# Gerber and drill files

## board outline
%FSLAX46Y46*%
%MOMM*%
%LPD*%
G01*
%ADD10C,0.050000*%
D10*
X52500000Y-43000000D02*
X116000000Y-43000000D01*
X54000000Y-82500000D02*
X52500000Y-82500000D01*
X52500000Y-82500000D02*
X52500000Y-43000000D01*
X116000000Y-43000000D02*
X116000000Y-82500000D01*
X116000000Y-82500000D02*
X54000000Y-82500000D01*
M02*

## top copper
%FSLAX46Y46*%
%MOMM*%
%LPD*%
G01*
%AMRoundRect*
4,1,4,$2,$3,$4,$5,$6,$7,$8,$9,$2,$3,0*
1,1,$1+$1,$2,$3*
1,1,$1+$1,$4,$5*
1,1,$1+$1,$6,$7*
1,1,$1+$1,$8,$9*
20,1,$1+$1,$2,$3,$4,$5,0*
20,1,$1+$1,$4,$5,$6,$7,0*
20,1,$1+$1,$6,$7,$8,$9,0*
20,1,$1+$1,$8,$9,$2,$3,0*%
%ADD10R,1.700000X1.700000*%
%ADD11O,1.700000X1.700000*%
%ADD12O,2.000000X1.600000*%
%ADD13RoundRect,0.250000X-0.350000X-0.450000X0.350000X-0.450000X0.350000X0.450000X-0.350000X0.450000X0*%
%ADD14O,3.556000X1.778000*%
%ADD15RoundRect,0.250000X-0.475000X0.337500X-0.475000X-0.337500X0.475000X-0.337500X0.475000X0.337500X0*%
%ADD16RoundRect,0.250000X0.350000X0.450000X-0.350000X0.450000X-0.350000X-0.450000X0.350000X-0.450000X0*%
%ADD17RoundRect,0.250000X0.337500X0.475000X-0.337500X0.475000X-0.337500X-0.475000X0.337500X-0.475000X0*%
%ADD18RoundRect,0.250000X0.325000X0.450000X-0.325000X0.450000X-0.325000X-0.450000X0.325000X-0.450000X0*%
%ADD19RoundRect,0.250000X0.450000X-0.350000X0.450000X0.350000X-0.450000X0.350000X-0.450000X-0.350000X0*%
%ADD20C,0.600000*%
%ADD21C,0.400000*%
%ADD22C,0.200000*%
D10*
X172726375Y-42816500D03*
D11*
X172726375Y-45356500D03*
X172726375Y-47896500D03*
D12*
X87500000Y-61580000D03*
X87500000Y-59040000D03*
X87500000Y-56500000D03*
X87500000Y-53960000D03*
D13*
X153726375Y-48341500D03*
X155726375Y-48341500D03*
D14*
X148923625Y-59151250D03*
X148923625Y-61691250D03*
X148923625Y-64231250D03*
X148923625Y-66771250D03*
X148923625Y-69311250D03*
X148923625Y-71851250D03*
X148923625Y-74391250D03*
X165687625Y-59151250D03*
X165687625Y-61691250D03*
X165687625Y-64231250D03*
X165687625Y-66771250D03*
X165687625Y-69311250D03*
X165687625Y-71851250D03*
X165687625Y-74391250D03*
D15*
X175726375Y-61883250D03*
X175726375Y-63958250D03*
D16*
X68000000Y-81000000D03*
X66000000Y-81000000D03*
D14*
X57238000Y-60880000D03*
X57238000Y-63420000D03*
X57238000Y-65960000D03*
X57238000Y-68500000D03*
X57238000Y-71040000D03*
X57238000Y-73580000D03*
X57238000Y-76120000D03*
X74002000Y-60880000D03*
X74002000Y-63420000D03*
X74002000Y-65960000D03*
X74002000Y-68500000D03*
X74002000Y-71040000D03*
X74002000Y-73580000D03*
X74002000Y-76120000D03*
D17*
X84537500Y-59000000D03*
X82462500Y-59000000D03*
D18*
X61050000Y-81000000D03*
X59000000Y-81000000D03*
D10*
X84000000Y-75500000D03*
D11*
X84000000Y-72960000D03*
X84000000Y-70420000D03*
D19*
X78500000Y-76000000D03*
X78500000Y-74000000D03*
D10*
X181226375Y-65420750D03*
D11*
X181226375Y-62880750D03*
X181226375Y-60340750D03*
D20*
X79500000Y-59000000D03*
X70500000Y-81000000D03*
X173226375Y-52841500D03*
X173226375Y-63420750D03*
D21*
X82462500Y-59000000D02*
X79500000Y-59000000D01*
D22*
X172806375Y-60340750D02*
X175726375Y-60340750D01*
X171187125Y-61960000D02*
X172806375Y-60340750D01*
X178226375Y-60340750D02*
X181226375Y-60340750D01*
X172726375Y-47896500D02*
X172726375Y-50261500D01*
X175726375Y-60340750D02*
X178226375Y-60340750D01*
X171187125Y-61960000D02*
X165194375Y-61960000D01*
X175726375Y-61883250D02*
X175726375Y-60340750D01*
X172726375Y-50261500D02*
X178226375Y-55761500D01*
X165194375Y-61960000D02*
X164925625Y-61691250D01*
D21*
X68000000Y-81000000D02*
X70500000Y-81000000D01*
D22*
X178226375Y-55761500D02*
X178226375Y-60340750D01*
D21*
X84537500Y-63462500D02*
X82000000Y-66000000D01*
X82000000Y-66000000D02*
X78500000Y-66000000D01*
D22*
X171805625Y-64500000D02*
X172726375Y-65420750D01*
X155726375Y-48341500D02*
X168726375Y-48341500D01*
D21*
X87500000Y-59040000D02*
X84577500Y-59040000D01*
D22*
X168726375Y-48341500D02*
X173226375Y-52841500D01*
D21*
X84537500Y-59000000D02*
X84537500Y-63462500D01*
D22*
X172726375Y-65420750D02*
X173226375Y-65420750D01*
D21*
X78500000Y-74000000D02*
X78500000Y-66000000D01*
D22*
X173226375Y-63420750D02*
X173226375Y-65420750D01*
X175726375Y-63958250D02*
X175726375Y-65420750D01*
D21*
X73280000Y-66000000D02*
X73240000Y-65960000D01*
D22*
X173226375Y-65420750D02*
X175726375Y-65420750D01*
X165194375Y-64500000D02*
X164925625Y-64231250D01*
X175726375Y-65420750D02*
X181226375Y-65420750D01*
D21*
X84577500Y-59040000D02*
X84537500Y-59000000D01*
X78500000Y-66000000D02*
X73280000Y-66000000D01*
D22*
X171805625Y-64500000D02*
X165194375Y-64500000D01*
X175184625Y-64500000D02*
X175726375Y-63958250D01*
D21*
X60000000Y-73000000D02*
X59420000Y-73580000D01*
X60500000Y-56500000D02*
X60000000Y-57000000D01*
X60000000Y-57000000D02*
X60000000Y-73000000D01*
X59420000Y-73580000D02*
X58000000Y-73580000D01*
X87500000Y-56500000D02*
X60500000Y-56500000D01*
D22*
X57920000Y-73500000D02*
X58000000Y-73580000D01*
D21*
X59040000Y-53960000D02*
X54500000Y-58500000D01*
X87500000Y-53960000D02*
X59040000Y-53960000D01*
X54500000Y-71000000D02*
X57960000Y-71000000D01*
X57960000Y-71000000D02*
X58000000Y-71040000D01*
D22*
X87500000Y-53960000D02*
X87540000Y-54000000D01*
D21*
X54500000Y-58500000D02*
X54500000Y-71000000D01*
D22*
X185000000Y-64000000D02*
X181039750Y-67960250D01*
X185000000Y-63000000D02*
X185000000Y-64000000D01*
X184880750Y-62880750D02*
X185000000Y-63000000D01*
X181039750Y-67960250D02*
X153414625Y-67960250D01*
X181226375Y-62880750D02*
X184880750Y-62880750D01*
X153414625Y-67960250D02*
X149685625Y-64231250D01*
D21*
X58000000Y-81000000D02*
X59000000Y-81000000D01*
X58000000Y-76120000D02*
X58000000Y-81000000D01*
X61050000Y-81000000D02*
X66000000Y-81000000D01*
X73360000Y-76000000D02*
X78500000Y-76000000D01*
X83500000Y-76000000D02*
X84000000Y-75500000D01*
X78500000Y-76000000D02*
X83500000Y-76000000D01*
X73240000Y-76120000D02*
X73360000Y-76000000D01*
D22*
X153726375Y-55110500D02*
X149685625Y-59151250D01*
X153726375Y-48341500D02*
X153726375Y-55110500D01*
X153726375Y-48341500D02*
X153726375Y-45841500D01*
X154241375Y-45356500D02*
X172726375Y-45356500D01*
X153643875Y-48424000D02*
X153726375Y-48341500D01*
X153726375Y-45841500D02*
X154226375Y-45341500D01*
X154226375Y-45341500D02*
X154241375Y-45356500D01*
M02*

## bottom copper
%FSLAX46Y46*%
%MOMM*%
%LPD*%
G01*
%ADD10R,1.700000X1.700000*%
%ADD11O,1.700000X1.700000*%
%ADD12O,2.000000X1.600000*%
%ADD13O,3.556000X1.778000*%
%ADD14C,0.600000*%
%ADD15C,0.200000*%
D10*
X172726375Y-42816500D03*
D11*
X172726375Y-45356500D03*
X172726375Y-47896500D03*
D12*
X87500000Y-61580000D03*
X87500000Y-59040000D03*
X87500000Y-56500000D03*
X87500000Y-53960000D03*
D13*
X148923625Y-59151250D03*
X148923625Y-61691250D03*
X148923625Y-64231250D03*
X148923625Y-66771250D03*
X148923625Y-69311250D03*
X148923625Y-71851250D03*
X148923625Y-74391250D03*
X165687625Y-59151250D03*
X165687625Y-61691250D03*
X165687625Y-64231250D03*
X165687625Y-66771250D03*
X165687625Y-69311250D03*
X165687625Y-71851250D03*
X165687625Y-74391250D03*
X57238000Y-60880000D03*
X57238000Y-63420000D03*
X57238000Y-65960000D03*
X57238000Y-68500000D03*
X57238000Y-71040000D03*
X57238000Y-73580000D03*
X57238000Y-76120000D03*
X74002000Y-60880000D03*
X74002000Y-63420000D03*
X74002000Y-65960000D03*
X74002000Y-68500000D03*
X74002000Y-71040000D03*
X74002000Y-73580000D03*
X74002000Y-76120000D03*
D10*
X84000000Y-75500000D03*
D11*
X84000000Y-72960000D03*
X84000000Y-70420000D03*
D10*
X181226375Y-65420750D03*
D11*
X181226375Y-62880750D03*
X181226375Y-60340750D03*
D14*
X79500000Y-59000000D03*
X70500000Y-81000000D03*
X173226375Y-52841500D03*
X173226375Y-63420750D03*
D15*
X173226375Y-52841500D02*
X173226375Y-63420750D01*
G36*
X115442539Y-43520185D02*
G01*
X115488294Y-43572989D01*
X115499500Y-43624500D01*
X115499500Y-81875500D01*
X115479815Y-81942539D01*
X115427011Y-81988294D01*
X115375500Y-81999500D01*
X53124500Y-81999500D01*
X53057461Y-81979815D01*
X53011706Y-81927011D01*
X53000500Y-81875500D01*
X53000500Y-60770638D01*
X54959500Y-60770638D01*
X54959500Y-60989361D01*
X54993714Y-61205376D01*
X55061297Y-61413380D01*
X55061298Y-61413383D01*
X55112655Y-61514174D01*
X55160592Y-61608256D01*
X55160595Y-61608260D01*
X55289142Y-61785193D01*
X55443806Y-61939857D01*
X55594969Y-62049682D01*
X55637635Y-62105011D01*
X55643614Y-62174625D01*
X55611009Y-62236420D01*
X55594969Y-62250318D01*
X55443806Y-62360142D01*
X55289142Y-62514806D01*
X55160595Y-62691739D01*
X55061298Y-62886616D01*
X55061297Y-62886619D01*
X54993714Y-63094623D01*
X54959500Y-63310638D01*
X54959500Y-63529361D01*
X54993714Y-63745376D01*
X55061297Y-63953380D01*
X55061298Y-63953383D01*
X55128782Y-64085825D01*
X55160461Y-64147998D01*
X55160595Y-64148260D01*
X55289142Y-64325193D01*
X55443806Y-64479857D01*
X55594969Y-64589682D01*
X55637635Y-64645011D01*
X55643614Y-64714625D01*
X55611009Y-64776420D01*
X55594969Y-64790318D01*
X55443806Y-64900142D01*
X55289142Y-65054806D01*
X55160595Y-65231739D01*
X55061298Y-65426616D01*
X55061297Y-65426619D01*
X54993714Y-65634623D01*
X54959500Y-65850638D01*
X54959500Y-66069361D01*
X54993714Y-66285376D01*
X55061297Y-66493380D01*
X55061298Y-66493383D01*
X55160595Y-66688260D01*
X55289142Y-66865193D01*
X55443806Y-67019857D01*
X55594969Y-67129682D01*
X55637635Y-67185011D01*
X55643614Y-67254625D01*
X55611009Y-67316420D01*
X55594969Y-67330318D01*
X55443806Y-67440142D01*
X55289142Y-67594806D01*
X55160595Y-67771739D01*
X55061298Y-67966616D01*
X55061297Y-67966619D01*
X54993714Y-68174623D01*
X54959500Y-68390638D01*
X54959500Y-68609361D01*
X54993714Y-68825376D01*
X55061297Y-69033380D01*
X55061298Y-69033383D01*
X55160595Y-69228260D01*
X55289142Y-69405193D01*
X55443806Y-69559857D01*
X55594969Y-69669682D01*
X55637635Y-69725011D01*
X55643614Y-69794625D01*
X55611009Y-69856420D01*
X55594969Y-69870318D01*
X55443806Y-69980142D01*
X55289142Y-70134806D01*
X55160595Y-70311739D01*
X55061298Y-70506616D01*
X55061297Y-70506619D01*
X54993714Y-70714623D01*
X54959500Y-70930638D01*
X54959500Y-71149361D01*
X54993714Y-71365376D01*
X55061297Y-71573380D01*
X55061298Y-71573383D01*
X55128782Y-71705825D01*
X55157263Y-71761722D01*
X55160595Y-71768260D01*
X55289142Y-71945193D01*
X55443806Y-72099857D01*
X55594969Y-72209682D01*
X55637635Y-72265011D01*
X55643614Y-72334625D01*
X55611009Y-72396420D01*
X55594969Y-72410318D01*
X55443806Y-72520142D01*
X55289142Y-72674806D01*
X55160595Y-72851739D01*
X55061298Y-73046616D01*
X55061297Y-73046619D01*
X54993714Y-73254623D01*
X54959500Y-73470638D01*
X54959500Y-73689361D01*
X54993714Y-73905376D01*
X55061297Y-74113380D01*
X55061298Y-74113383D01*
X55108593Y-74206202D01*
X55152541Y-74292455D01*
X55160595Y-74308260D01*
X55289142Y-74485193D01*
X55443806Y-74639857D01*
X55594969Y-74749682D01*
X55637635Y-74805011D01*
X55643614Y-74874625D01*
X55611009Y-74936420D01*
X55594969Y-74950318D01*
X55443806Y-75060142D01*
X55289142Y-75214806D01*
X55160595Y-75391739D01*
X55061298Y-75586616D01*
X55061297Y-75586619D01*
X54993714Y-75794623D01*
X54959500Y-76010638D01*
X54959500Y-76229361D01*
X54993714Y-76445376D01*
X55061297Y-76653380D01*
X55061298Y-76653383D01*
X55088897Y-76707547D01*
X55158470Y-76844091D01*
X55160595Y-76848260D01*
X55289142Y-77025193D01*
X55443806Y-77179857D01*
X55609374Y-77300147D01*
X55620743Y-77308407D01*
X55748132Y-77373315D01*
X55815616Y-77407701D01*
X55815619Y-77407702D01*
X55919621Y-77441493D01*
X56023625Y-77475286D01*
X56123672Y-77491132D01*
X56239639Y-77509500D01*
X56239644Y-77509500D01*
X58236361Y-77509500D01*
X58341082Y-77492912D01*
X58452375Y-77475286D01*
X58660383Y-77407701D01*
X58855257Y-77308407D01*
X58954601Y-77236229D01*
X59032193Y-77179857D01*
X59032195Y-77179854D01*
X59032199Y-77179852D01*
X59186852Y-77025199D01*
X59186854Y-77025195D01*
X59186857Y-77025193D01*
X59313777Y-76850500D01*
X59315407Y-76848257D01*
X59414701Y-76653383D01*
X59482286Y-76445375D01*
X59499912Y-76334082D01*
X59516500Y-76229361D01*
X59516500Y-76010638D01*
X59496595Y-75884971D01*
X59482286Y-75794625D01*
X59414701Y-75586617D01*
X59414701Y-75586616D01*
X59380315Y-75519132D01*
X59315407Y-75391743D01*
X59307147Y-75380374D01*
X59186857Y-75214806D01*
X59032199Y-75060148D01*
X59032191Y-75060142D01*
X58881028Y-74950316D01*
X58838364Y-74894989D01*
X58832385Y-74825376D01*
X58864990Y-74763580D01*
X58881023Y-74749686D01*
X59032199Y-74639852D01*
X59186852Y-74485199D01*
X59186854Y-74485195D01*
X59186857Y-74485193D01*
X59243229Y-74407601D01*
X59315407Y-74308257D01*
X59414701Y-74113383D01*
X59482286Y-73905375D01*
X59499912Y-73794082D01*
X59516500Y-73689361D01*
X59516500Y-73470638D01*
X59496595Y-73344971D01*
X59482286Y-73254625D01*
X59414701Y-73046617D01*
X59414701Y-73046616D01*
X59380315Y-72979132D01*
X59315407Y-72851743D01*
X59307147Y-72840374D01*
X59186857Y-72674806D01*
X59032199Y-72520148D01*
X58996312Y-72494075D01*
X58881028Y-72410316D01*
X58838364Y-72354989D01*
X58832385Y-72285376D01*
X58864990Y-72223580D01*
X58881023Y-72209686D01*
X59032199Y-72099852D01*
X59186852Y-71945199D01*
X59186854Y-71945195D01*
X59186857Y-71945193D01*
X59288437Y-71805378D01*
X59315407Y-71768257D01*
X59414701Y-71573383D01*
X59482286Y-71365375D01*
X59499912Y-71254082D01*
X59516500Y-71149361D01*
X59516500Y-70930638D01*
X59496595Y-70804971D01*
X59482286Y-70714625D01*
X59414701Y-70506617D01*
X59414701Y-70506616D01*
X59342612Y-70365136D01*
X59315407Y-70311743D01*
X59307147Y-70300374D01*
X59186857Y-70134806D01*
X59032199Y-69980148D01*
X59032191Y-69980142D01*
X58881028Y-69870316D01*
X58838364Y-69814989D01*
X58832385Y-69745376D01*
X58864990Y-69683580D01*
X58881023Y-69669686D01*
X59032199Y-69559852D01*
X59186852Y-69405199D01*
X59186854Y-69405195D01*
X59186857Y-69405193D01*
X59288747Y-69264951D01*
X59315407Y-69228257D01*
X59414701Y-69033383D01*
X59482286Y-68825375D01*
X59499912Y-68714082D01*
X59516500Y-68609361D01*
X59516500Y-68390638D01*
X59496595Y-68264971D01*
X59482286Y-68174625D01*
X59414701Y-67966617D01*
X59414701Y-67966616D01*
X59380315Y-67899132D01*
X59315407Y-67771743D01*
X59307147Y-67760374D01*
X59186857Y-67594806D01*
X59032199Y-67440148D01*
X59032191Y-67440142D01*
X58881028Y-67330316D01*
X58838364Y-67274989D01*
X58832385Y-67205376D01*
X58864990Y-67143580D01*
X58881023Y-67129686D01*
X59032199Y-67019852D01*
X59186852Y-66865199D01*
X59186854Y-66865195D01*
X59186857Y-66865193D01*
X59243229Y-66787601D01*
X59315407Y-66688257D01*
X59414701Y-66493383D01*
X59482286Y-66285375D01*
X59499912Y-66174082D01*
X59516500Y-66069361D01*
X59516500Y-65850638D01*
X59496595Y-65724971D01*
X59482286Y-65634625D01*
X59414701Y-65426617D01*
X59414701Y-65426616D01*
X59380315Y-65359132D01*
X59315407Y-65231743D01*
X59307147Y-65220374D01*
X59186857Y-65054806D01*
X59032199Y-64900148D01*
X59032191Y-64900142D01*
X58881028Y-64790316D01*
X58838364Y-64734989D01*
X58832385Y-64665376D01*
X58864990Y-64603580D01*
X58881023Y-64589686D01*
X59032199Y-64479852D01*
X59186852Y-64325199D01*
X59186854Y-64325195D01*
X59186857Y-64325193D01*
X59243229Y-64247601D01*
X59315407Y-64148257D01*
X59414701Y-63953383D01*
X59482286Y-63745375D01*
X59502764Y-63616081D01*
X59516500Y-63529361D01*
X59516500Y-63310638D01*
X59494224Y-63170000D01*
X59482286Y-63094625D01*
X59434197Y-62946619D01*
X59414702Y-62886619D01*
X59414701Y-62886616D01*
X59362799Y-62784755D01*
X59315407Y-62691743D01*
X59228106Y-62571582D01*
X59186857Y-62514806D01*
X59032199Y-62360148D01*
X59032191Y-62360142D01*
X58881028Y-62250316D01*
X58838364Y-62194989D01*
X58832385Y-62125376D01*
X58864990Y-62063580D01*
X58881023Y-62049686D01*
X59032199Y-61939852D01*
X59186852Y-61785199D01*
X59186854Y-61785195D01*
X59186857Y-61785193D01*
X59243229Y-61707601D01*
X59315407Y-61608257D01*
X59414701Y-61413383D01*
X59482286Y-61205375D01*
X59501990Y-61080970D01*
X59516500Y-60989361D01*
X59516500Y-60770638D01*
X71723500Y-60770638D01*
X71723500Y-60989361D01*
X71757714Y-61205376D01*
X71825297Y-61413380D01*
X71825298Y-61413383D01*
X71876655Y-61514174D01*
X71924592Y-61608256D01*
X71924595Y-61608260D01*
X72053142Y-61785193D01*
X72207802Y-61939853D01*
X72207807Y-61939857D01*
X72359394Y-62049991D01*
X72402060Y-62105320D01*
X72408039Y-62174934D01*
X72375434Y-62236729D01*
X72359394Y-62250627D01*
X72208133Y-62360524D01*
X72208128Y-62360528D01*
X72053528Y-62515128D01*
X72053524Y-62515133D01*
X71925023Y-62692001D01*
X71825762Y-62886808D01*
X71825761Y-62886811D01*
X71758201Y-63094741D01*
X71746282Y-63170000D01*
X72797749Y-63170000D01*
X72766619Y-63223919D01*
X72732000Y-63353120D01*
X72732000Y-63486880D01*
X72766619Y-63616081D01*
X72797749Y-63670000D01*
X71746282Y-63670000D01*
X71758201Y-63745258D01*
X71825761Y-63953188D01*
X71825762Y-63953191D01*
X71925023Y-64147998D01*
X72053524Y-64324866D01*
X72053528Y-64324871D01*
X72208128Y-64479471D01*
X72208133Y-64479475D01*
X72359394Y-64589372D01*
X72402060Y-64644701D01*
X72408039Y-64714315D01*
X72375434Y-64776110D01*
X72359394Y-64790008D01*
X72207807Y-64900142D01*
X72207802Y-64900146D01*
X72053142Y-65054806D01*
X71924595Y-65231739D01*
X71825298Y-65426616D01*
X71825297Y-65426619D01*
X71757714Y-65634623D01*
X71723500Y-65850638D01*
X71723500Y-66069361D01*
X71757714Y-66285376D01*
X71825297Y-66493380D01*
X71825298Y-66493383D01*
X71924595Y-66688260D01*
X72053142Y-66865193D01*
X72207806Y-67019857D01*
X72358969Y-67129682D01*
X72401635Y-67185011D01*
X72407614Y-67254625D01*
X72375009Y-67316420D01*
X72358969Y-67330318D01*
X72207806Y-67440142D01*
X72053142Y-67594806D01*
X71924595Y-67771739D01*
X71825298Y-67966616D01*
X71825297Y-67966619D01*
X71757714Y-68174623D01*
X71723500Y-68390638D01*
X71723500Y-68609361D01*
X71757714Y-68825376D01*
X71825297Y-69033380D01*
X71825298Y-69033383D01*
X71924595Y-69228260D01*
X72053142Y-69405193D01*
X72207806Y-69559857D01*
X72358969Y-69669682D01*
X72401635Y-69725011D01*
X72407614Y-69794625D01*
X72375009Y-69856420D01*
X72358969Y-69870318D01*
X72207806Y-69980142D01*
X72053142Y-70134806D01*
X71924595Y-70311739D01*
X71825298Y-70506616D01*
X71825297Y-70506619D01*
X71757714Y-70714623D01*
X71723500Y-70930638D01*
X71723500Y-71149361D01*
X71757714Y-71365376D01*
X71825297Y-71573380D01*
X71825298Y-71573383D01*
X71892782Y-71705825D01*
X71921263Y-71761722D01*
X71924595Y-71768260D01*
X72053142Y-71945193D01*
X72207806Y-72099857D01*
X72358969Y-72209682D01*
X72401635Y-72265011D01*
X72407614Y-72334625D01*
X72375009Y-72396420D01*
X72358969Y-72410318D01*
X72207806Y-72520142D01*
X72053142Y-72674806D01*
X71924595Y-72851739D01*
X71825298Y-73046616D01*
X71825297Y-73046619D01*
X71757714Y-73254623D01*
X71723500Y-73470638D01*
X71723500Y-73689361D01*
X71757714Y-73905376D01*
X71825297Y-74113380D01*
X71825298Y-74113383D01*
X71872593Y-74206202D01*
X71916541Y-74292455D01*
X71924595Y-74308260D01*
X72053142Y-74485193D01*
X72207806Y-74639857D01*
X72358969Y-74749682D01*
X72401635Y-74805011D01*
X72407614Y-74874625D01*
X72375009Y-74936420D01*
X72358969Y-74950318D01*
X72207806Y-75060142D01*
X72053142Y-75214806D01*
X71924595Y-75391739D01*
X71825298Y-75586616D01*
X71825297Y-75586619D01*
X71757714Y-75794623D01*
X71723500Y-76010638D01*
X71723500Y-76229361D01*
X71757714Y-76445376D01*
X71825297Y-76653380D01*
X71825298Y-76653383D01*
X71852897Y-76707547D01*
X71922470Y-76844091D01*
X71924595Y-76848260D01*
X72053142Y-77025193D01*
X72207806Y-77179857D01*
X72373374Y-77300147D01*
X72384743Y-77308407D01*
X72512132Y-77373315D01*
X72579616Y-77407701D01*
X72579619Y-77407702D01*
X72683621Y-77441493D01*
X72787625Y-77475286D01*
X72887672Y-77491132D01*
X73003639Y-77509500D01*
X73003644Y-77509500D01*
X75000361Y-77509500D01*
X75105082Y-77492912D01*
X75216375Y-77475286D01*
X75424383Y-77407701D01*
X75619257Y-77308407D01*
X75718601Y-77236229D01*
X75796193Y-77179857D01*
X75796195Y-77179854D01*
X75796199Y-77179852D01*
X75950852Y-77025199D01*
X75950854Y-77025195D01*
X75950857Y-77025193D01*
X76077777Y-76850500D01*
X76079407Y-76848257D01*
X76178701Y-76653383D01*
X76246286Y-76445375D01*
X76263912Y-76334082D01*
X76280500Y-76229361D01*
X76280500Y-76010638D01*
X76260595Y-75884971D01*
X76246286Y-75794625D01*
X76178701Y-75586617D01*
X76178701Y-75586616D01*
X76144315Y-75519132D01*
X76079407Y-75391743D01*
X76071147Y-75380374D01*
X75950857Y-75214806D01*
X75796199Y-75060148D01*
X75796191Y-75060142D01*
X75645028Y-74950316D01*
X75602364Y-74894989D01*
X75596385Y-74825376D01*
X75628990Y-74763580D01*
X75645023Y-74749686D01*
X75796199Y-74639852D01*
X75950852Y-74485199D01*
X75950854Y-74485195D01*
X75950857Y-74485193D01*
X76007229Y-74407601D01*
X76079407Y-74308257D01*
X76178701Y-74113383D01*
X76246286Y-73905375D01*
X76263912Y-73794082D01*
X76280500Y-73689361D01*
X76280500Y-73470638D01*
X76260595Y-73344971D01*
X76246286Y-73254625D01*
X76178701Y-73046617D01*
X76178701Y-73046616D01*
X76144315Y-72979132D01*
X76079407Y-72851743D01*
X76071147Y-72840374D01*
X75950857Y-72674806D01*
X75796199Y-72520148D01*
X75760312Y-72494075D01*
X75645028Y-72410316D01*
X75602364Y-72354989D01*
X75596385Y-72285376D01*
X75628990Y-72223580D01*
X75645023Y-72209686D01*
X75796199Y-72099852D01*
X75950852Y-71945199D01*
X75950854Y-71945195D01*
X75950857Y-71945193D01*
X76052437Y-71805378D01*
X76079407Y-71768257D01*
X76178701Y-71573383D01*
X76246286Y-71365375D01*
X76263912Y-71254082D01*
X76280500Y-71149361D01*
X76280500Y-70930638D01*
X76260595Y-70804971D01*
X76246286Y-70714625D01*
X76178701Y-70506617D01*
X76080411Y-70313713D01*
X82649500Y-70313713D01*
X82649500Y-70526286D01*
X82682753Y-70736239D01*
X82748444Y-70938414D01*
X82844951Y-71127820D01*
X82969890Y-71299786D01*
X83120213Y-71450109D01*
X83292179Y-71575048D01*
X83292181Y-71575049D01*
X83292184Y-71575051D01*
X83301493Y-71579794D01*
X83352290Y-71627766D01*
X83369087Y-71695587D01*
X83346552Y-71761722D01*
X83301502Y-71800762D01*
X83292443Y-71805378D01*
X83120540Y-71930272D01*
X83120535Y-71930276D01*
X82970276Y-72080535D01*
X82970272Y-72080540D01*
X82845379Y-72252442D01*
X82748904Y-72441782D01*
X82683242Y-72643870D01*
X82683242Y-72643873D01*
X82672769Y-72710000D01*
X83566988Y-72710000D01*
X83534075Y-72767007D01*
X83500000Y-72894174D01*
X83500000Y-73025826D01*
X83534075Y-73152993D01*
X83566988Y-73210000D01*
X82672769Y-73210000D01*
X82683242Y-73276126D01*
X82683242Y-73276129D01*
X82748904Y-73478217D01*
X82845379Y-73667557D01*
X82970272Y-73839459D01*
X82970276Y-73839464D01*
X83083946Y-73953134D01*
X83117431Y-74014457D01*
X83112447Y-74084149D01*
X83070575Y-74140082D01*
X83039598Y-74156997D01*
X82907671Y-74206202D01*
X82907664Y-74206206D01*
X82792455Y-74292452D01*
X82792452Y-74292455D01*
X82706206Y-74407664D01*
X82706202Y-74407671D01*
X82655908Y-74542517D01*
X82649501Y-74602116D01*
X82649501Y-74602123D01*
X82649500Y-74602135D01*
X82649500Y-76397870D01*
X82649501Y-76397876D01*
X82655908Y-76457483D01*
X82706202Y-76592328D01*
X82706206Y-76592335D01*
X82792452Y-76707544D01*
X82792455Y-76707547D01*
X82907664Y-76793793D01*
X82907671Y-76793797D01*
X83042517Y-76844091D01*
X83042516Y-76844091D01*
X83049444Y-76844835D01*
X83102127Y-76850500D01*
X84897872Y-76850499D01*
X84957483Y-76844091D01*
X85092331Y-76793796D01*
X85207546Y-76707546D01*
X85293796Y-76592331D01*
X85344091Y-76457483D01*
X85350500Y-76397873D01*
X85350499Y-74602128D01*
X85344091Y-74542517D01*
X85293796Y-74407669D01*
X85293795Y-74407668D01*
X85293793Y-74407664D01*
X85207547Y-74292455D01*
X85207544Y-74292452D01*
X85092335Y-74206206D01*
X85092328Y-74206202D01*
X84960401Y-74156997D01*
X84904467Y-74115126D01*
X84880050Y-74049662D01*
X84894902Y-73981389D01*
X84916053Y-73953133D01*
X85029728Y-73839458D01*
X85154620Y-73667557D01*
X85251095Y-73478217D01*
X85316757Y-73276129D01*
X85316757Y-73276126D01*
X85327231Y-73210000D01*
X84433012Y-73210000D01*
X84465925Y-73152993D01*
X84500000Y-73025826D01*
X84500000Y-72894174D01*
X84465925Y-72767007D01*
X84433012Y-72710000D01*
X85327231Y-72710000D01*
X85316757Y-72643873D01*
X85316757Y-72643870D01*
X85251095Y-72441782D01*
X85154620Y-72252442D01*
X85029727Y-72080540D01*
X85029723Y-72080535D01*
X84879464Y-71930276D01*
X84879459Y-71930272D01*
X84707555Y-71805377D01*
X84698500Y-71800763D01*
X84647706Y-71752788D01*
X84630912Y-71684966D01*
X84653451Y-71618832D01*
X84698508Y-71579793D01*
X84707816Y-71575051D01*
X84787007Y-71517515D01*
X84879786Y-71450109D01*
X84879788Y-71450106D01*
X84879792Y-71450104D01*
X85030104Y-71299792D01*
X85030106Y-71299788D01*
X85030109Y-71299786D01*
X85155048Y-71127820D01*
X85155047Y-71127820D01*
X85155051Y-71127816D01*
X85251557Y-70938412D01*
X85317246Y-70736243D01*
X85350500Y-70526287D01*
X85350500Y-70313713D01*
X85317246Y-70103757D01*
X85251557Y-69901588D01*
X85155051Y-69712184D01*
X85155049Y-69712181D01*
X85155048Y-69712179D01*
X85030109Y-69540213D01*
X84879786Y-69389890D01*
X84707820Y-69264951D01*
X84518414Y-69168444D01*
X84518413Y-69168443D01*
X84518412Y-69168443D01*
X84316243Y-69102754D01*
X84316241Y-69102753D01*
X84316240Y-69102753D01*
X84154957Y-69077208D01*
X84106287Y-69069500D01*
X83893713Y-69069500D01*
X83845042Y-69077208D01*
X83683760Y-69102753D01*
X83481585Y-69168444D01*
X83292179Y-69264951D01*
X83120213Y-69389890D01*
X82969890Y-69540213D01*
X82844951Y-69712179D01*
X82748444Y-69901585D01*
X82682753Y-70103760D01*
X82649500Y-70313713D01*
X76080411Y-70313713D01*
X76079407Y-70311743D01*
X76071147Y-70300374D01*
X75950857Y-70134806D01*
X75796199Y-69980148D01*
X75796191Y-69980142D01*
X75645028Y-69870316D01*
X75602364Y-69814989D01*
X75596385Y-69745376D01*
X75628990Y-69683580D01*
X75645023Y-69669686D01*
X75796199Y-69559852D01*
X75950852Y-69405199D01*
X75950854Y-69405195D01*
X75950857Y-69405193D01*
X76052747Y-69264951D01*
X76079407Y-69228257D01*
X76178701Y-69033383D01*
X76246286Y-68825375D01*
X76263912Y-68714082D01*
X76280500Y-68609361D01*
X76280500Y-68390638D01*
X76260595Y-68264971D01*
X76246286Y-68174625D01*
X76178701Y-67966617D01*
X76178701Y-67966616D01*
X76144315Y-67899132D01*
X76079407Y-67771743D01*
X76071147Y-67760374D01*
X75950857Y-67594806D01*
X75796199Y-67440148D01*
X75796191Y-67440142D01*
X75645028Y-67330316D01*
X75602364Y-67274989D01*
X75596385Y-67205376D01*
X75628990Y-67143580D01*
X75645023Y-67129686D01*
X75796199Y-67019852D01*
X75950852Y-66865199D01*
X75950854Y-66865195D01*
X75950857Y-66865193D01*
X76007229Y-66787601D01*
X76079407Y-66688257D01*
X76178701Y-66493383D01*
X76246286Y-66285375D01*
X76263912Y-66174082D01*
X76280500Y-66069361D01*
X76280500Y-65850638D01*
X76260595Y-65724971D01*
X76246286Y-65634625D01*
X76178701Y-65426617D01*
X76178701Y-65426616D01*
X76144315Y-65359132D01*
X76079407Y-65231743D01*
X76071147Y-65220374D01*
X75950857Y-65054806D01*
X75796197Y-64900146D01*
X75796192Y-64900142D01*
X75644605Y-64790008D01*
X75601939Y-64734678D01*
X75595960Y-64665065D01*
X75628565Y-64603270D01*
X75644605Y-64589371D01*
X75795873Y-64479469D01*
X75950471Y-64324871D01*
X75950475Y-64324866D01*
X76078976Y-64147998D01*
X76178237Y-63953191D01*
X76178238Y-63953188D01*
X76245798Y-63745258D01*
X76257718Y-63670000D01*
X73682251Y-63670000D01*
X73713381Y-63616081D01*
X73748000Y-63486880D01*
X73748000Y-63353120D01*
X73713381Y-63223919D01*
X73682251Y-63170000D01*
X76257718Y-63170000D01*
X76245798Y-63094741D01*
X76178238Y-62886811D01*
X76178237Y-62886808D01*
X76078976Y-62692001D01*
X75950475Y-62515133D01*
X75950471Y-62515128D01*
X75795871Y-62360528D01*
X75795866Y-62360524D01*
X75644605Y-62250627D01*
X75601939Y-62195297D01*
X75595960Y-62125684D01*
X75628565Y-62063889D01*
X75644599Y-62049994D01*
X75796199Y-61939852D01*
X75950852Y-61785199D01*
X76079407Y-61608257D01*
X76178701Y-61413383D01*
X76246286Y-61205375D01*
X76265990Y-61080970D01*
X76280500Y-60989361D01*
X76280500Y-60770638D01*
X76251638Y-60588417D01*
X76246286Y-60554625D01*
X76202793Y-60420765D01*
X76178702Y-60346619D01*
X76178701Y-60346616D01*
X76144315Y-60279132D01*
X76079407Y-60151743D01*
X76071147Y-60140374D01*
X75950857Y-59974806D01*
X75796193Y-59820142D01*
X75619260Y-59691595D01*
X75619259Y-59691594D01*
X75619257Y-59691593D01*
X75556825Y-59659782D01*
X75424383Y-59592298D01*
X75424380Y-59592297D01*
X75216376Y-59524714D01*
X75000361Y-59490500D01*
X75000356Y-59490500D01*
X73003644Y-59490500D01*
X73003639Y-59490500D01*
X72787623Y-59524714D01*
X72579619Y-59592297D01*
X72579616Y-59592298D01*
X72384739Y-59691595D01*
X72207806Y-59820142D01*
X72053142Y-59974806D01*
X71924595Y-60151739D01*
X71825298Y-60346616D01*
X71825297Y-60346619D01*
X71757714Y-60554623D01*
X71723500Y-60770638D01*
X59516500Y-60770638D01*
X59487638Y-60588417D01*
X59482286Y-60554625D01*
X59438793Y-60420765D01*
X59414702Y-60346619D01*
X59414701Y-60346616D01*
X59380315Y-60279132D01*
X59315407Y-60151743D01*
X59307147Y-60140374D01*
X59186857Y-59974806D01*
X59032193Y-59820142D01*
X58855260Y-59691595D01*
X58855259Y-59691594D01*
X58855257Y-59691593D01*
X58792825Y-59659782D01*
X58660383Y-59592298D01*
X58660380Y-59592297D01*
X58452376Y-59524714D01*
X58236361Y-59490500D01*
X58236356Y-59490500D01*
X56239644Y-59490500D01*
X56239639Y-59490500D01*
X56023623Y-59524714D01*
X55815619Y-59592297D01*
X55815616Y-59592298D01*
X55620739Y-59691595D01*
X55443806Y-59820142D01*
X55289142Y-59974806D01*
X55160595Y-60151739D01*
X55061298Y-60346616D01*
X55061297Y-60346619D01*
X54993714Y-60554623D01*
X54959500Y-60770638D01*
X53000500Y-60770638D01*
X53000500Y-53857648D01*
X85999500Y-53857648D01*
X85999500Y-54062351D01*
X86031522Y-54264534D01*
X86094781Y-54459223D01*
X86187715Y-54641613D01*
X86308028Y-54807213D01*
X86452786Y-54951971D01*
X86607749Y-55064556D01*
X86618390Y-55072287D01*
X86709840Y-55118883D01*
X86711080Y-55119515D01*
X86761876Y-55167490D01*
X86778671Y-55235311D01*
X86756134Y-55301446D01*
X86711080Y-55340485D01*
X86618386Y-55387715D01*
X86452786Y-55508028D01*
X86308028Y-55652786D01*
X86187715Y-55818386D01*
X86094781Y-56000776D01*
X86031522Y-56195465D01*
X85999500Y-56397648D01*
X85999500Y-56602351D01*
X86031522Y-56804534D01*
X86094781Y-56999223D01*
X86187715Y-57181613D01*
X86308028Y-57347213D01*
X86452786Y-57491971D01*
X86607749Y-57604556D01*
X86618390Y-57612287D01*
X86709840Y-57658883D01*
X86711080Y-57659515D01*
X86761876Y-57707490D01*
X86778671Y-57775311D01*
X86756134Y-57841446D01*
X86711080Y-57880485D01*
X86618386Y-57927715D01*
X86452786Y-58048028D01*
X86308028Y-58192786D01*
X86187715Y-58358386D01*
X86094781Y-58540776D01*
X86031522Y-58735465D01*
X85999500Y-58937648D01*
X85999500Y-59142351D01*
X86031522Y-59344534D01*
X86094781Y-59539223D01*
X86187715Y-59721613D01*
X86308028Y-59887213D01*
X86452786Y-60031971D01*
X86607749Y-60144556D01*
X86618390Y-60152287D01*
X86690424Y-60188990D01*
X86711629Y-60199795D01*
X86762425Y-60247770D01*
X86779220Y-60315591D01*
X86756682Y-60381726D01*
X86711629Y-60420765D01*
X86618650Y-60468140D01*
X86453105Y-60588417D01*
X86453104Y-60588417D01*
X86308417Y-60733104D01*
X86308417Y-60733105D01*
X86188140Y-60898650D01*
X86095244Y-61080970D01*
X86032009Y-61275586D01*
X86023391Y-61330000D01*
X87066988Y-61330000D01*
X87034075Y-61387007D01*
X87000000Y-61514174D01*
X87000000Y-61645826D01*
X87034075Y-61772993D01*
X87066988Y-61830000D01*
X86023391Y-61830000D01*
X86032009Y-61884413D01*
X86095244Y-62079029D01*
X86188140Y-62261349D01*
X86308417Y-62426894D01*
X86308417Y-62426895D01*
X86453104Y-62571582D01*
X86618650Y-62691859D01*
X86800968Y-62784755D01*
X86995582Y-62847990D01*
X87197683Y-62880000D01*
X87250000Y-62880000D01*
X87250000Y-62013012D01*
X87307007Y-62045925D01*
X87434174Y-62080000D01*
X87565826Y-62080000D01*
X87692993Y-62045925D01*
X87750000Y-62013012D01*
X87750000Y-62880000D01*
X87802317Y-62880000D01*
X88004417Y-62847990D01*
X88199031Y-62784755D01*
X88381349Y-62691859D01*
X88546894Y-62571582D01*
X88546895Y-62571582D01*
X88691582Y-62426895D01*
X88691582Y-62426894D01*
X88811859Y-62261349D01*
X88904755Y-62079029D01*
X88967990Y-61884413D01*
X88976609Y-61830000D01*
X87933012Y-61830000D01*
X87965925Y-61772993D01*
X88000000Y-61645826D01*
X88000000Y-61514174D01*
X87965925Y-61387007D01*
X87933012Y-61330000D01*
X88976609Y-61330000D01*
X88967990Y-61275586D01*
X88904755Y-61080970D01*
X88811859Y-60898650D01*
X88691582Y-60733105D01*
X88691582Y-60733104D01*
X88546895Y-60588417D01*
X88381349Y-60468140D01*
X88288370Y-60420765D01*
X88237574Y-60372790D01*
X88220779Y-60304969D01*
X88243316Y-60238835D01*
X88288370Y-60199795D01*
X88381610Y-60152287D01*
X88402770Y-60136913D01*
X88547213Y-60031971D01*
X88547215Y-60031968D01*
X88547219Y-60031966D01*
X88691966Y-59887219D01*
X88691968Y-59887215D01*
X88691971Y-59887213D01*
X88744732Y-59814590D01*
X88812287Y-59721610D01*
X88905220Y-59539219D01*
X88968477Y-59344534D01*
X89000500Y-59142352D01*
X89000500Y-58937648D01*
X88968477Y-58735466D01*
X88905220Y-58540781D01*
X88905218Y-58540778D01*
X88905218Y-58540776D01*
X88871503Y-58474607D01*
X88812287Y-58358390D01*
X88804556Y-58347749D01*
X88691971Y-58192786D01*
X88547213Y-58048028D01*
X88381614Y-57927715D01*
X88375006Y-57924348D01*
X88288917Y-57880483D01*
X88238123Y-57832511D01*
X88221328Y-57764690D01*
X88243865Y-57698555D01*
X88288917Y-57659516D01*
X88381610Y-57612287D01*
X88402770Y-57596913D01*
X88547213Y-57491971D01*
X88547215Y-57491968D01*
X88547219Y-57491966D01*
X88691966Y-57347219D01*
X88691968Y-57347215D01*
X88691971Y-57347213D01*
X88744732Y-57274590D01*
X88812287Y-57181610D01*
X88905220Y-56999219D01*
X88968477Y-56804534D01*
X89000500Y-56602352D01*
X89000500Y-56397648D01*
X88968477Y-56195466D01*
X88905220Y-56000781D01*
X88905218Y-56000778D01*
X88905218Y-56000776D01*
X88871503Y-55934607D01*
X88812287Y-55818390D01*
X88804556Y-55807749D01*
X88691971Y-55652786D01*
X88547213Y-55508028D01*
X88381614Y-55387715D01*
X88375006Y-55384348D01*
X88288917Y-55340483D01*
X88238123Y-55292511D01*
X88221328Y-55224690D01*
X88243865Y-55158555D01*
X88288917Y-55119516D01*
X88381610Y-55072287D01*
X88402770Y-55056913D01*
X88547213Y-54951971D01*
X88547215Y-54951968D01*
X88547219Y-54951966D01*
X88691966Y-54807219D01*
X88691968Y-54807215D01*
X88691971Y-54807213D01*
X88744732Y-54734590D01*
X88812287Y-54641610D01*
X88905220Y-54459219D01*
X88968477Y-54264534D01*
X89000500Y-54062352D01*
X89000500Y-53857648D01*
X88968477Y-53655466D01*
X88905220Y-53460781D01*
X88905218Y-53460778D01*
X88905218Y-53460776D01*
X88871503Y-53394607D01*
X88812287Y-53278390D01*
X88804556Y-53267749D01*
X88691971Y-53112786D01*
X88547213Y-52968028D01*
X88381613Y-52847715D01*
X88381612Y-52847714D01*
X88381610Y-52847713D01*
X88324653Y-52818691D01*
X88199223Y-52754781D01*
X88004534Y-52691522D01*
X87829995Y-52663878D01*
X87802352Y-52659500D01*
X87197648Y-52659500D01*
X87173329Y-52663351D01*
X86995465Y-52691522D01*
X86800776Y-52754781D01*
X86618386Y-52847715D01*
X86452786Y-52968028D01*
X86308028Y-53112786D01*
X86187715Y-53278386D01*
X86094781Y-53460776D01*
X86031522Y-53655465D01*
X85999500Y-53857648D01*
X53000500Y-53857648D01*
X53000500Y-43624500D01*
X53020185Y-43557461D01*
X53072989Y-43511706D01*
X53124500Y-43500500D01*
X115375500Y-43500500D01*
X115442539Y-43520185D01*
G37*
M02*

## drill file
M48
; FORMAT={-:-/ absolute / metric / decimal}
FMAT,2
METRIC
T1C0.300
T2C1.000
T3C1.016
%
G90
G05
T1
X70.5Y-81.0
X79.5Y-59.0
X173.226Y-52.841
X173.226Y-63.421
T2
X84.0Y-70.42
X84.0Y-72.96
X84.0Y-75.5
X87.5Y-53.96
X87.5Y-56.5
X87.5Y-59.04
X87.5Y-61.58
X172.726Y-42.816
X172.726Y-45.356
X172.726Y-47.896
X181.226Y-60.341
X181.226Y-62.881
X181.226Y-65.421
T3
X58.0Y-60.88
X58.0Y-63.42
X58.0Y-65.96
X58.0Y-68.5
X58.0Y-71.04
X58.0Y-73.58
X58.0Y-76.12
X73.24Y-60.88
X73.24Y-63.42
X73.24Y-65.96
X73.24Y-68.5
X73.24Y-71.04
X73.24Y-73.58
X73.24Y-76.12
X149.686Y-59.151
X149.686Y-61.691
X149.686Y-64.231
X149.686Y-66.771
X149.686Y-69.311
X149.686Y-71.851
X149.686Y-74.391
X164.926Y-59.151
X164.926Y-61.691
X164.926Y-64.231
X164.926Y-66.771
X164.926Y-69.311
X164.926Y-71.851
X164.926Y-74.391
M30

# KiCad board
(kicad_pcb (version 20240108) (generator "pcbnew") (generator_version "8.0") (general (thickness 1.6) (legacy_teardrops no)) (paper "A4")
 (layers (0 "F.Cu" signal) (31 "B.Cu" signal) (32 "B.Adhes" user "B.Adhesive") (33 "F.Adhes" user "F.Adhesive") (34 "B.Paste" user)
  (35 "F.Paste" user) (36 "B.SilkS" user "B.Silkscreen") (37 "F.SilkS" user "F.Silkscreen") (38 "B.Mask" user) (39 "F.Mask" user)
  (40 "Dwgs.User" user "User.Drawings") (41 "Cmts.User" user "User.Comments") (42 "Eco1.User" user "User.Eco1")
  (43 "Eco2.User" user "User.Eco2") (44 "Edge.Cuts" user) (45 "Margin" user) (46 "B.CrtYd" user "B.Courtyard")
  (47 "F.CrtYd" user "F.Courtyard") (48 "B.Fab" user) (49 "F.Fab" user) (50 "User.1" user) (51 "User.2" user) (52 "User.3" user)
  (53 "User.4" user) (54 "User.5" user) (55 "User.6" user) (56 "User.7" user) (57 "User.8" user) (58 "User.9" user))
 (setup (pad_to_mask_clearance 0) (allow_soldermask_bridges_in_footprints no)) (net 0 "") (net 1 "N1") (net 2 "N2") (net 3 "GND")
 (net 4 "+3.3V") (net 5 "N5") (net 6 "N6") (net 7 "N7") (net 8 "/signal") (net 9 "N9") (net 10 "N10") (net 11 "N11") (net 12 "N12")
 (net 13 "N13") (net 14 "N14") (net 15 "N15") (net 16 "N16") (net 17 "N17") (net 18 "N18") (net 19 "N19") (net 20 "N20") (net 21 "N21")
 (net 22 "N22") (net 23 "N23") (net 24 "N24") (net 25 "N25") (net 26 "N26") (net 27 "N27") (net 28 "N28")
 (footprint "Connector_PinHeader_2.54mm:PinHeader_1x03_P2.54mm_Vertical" (layer "F.Cu") (at 172.726375 42.8165)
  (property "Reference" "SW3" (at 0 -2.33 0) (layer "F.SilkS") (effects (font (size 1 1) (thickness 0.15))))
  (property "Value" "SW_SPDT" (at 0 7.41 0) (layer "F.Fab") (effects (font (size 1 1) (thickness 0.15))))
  (pad "1" thru_hole rect (at 0 0) (size 1.7 1.7) (drill 1) (layers "*.Cu" "*.Mask") (remove_unused_layers no) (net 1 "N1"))
  (pad "2" thru_hole oval (at 0 2.54) (size 1.7 1.7) (drill 1) (layers "*.Cu" "*.Mask") (remove_unused_layers no) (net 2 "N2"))
  (pad "3" thru_hole oval (at 0 5.08) (size 1.7 1.7) (drill 1) (layers "*.Cu" "*.Mask") (remove_unused_layers no) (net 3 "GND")))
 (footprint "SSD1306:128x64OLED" (layer "F.Cu") (at 98.1 57.96 90)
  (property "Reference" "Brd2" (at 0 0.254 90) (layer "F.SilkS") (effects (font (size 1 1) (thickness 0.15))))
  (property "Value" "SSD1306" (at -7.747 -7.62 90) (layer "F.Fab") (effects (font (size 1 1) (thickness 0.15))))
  (pad "1" thru_hole oval (at -3.62 -10.6 180) (size 2 1.6) (drill 1) (layers "*.Cu" "*.Mask") (remove_unused_layers no) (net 3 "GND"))
  (pad "2" thru_hole oval (at -1.08 -10.6 180) (size 2 1.6) (drill 1) (layers "*.Cu" "*.Mask") (remove_unused_layers no) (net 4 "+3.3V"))
  (pad "3" thru_hole oval (at 1.46 -10.6 180) (size 2 1.6) (drill 1) (layers "*.Cu" "*.Mask") (remove_unused_layers no) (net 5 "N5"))
  (pad "4" thru_hole oval (at 4 -10.6 180) (size 2 1.6) (drill 1) (layers "*.Cu" "*.Mask") (remove_unused_layers no) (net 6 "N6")))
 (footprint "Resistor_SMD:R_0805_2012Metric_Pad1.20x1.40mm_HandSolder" (layer "F.Cu") (at 154.726375 48.3415)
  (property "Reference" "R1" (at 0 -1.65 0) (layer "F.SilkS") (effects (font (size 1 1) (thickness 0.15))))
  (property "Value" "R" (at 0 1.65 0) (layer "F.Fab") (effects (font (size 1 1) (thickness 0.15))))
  (pad "1" smd roundrect (at -1 0) (size 1.2 1.4) (layers "F.Cu" "F.Paste" "F.Mask") (roundrect_rratio 0.208333) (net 2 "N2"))
  (pad "2" smd roundrect (at 1 0) (size 1.2 1.4) (layers "F.Cu" "F.Paste" "F.Mask") (roundrect_rratio 0.208333) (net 4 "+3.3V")))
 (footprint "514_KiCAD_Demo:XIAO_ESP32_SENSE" (layer "F.Cu") (at 157.305625 66.77125)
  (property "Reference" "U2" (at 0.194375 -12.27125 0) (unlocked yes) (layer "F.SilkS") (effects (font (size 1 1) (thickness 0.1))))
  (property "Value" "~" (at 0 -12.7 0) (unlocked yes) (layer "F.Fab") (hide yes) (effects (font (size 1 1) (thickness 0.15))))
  (pad "1" thru_hole oval (at -7.62 -7.62) (size 3.556 1.778) (drill 1.016 (offset -0.762 0)) (layers "*.Cu" "*.Mask")
   (remove_unused_layers no) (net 2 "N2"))
  (pad "2" thru_hole oval (at -7.62 -5.08) (size 3.556 1.778) (drill 1.016 (offset -0.762 0)) (layers "*.Cu" "*.Mask")
   (remove_unused_layers no) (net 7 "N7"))
  (pad "3" thru_hole oval (at -7.62 -2.54) (size 3.556 1.778) (drill 1.016 (offset -0.762 0)) (layers "*.Cu" "*.Mask")
   (remove_unused_layers no) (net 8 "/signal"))
  (pad "4" thru_hole oval (at -7.62 0) (size 3.556 1.778) (drill 1.016 (offset -0.762 0)) (layers "*.Cu" "*.Mask") (remove_unused_layers no)
   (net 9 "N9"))
  (pad "5" thru_hole oval (at -7.62 2.54) (size 3.556 1.778) (drill 1.016 (offset -0.762 0)) (layers "*.Cu" "*.Mask")
   (remove_unused_layers no) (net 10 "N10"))
  (pad "6" thru_hole oval (at -7.62 5.08) (size 3.556 1.778) (drill 1.016 (offset -0.762 0)) (layers "*.Cu" "*.Mask")
   (remove_unused_layers no) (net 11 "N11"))
  (pad "7" thru_hole oval (at -7.62 7.62) (size 3.556 1.778) (drill 1.016 (offset -0.762 0)) (layers "*.Cu" "*.Mask")
   (remove_unused_layers no) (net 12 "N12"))
  (pad "8" thru_hole oval (at 7.62 -7.62) (size 3.556 1.778) (drill 1.016 (offset 0.762 0)) (layers "*.Cu" "*.Mask")
   (remove_unused_layers no) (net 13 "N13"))
  (pad "9" thru_hole oval (at 7.62 -5.08) (size 3.556 1.778) (drill 1.016 (offset 0.762 0)) (layers "*.Cu" "*.Mask")
   (remove_unused_layers no) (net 3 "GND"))
  (pad "10" thru_hole oval (at 7.62 -2.54) (size 3.556 1.778) (drill 1.016 (offset 0.762 0)) (layers "*.Cu" "*.Mask")
   (remove_unused_layers no) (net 4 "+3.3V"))
  (pad "11" thru_hole oval (at 7.62 0) (size 3.556 1.778) (drill 1.016 (offset 0.762 0)) (layers "*.Cu" "*.Mask") (remove_unused_layers no)
   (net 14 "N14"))
  (pad "12" thru_hole oval (at 7.62 2.54) (size 3.556 1.778) (drill 1.016 (offset 0.762 0)) (layers "*.Cu" "*.Mask")
   (remove_unused_layers no) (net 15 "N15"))
  (pad "13" thru_hole oval (at 7.62 5.08) (size 3.556 1.778) (drill 1.016 (offset 0.762 0)) (layers "*.Cu" "*.Mask")
   (remove_unused_layers no) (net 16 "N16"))
  (pad "14" thru_hole oval (at 7.62 7.62) (size 3.556 1.778) (drill 1.016 (offset 0.762 0)) (layers "*.Cu" "*.Mask")
   (remove_unused_layers no) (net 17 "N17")))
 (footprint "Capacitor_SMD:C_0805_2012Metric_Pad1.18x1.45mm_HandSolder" (layer "F.Cu") (at 175.726375 62.92075 -90)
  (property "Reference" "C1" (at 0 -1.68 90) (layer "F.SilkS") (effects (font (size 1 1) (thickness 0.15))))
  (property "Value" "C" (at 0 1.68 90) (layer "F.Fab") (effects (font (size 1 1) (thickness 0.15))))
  (pad "1" smd roundrect (at -1.0375 0 270) (size 1.175 1.45) (layers "F.Cu" "F.Paste" "F.Mask") (roundrect_rratio 0.212766) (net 3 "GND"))
  (pad "2" smd roundrect (at 1.0375 0 270) (size 1.175 1.45) (layers "F.Cu" "F.Paste" "F.Mask") (roundrect_rratio 0.212766) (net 4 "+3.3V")))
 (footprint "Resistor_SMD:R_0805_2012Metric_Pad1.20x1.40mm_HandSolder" (layer "F.Cu") (at 67 81 180)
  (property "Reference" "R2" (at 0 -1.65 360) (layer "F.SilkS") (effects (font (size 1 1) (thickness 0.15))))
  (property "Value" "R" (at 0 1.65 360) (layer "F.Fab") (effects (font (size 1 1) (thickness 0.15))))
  (pad "1" smd roundrect (at -1 0 180) (size 1.2 1.4) (layers "F.Cu" "F.Paste" "F.Mask") (roundrect_rratio 0.208333) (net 3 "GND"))
  (pad "2" smd roundrect (at 1 0 180) (size 1.2 1.4) (layers "F.Cu" "F.Paste" "F.Mask") (roundrect_rratio 0.208333) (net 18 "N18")))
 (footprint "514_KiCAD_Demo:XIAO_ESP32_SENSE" (layer "F.Cu") (at 65.62 68.5)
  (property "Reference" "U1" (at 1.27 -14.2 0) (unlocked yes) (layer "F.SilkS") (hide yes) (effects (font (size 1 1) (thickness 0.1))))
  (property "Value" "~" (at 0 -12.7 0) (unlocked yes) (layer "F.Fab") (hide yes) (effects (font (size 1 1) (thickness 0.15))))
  (pad "1" thru_hole oval (at -7.62 -7.62) (size 3.556 1.778) (drill 1.016 (offset -0.762 0)) (layers "*.Cu" "*.Mask")
   (remove_unused_layers no) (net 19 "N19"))
  (pad "2" thru_hole oval (at -7.62 -5.08) (size 3.556 1.778) (drill 1.016 (offset -0.762 0)) (layers "*.Cu" "*.Mask")
   (remove_unused_layers no) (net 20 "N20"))
  (pad "3" thru_hole oval (at -7.62 -2.54) (size 3.556 1.778) (drill 1.016 (offset -0.762 0)) (layers "*.Cu" "*.Mask")
   (remove_unused_layers no) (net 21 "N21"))
  (pad "4" thru_hole oval (at -7.62 0) (size 3.556 1.778) (drill 1.016 (offset -0.762 0)) (layers "*.Cu" "*.Mask") (remove_unused_layers no)
   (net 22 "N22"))
  (pad "5" thru_hole oval (at -7.62 2.54) (size 3.556 1.778) (drill 1.016 (offset -0.762 0)) (layers "*.Cu" "*.Mask")
   (remove_unused_layers no) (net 6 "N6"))
  (pad "6" thru_hole oval (at -7.62 5.08) (size 3.556 1.778) (drill 1.016 (offset -0.762 0)) (layers "*.Cu" "*.Mask")
   (remove_unused_layers no) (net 5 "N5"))
  (pad "7" thru_hole oval (at -7.62 7.62) (size 3.556 1.778) (drill 1.016 (offset -0.762 0)) (layers "*.Cu" "*.Mask")
   (remove_unused_layers no) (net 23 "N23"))
  (pad "8" thru_hole oval (at 7.62 -7.62) (size 3.556 1.778) (drill 1.016 (offset 0.762 0)) (layers "*.Cu" "*.Mask")
   (remove_unused_layers no) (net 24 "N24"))
  (pad "9" thru_hole oval (at 7.62 -5.08) (size 3.556 1.778) (drill 1.016 (offset 0.762 0)) (layers "*.Cu" "*.Mask")
   (remove_unused_layers no) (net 3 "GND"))
  (pad "10" thru_hole oval (at 7.62 -2.54) (size 3.556 1.778) (drill 1.016 (offset 0.762 0)) (layers "*.Cu" "*.Mask")
   (remove_unused_layers no) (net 4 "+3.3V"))
  (pad "11" thru_hole oval (at 7.62 0) (size 3.556 1.778) (drill 1.016 (offset 0.762 0)) (layers "*.Cu" "*.Mask") (remove_unused_layers no)
   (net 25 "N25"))
  (pad "12" thru_hole oval (at 7.62 2.54) (size 3.556 1.778) (drill 1.016 (offset 0.762 0)) (layers "*.Cu" "*.Mask")
   (remove_unused_layers no) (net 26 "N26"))
  (pad "13" thru_hole oval (at 7.62 5.08) (size 3.556 1.778) (drill 1.016 (offset 0.762 0)) (layers "*.Cu" "*.Mask")
   (remove_unused_layers no) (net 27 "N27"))
  (pad "14" thru_hole oval (at 7.62 7.62) (size 3.556 1.778) (drill 1.016 (offset 0.762 0)) (layers "*.Cu" "*.Mask")
   (remove_unused_layers no) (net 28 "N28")))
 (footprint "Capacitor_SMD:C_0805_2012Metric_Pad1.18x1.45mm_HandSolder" (layer "F.Cu") (at 83.5 59 180)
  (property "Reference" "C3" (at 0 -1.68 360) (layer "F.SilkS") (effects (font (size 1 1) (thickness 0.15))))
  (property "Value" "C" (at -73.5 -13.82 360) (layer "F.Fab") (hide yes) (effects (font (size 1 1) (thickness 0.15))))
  (pad "1" smd roundrect (at -1.0375 0 180) (size 1.175 1.45) (layers "F.Cu" "F.Paste" "F.Mask") (roundrect_rratio 0.212766) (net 4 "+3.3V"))
  (pad "2" smd roundrect (at 1.0375 0 180) (size 1.175 1.45) (layers "F.Cu" "F.Paste" "F.Mask") (roundrect_rratio 0.212766) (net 3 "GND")))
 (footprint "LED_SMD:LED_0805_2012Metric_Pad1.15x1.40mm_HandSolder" (layer "F.Cu") (at 60.025 81 180)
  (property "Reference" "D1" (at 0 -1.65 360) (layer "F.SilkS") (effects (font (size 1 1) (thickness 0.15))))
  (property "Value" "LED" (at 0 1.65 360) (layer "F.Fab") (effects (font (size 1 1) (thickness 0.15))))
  (pad "1" smd roundrect (at -1.025 0 180) (size 1.15 1.4) (layers "F.Cu" "F.Paste" "F.Mask") (roundrect_rratio 0.217391) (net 18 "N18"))
  (pad "2" smd roundrect (at 1.025 0 180) (size 1.15 1.4) (layers "F.Cu" "F.Paste" "F.Mask") (roundrect_rratio 0.217391) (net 23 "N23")))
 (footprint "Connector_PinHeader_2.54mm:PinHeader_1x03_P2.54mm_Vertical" (layer "F.Cu") (at 84 75.5 180)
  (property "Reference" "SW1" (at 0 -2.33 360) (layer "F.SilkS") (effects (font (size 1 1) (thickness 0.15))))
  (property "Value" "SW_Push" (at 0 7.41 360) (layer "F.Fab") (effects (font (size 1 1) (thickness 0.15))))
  (pad "1" thru_hole rect (at 0 0 180) (size 1.7 1.7) (drill 1) (layers "*.Cu" "*.Mask") (remove_unused_layers no) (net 28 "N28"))
  (pad "2" thru_hole oval (at 0 2.54 180) (size 1.7 1.7) (drill 1) (layers "*.Cu" "*.Mask") (remove_unused_layers no) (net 3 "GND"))
  (pad "3" thru_hole oval (at 0 5.08 180) (size 1.7 1.7) (drill 1) (layers "*.Cu" "*.Mask") (remove_unused_layers no)))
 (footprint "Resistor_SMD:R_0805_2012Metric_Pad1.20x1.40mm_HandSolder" (layer "F.Cu") (at 78.5 75 90)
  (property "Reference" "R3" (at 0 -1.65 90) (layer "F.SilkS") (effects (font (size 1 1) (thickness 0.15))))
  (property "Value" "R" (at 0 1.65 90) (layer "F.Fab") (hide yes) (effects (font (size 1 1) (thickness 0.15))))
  (pad "1" smd roundrect (at -1 0 90) (size 1.2 1.4) (layers "F.Cu" "F.Paste" "F.Mask") (roundrect_rratio 0.208333) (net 28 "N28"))
  (pad "2" smd roundrect (at 1 0 90) (size 1.2 1.4) (layers "F.Cu" "F.Paste" "F.Mask") (roundrect_rratio 0.208333) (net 4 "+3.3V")))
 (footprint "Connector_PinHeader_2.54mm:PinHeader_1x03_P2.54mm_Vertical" (layer "F.Cu") (at 181.226375 65.42075 180)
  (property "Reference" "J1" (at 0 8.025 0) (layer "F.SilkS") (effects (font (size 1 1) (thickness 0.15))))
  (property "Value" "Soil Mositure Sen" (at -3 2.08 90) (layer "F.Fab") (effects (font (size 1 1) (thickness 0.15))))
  (pad "1" thru_hole rect (at 0 0 180) (size 1.7 1.7) (drill 1) (layers "*.Cu" "*.Mask") (remove_unused_layers no) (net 4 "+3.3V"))
  (pad "2" thru_hole oval (at 0 2.54 180) (size 1.7 1.7) (drill 1) (layers "*.Cu" "*.Mask") (remove_unused_layers no) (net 8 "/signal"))
  (pad "3" thru_hole oval (at 0 5.08 180) (size 1.7 1.7) (drill 1) (layers "*.Cu" "*.Mask") (remove_unused_layers no) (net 3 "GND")))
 (gr_line (start 52.5 43) (end 116 43) (stroke (width 0.05) (type default)) (layer "Edge.Cuts"))
 (gr_line (start 54 82.5) (end 52.5 82.5) (stroke (width 0.05) (type default)) (layer "Edge.Cuts"))
 (gr_line (start 52.5 82.5) (end 52.5 43) (stroke (width 0.05) (type default)) (layer "Edge.Cuts"))
 (gr_line (start 116 43) (end 116 82.5) (stroke (width 0.05) (type default)) (layer "Edge.Cuts"))
 (gr_line (start 116 82.5) (end 54 82.5) (stroke (width 0.05) (type default)) (layer "Edge.Cuts"))
 (segment (start 82.4625 59) (end 79.5 59) (width 0.4) (layer "F.Cu") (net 3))
 (segment (start 172.806375 60.34075) (end 175.726375 60.34075) (width 0.2) (layer "F.Cu") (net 3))
 (segment (start 171.187125 61.96) (end 172.806375 60.34075) (width 0.2) (layer "F.Cu") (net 3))
 (segment (start 178.226375 60.34075) (end 181.226375 60.34075) (width 0.2) (layer "F.Cu") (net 3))
 (segment (start 172.726375 47.8965) (end 172.726375 50.2615) (width 0.2) (layer "F.Cu") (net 3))
 (segment (start 175.726375 60.34075) (end 178.226375 60.34075) (width 0.2) (layer "F.Cu") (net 3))
 (segment (start 171.187125 61.96) (end 165.194375 61.96) (width 0.2) (layer "F.Cu") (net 3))
 (segment (start 175.726375 61.88325) (end 175.726375 60.34075) (width 0.2) (layer "F.Cu") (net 3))
 (segment (start 172.726375 50.2615) (end 178.226375 55.7615) (width 0.2) (layer "F.Cu") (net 3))
 (segment (start 165.194375 61.96) (end 164.925625 61.69125) (width 0.2) (layer "F.Cu") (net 3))
 (segment (start 68 81) (end 70.5 81) (width 0.4) (layer "F.Cu") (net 3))
 (segment (start 178.226375 55.7615) (end 178.226375 60.34075) (width 0.2) (layer "F.Cu") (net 3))
 (via (at 79.5 59) (size 0.6) (drill 0.3) (layers "F.Cu" "B.Cu") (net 3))
 (via (at 70.5 81) (size 0.6) (drill 0.3) (layers "F.Cu" "B.Cu") (free yes) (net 3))
 (segment (start 84.5375 63.4625) (end 82 66) (width 0.4) (layer "F.Cu") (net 4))
 (segment (start 82 66) (end 78.5 66) (width 0.4) (layer "F.Cu") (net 4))
 (segment (start 171.805625 64.5) (end 172.726375 65.42075) (width 0.2) (layer "F.Cu") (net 4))
 (segment (start 155.726375 48.3415) (end 168.726375 48.3415) (width 0.2) (layer "F.Cu") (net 4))
 (segment (start 87.5 59.04) (end 84.5775 59.04) (width 0.4) (layer "F.Cu") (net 4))
 (segment (start 168.726375 48.3415) (end 173.226375 52.8415) (width 0.2) (layer "F.Cu") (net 4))
 (segment (start 84.5375 59) (end 84.5375 63.4625) (width 0.4) (layer "F.Cu") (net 4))
 (segment (start 172.726375 65.42075) (end 173.226375 65.42075) (width 0.2) (layer "F.Cu") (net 4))
 (segment (start 78.5 74) (end 78.5 66) (width 0.4) (layer "F.Cu") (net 4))
 (segment (start 173.226375 63.42075) (end 173.226375 65.42075) (width 0.2) (layer "F.Cu") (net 4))
 (segment (start 175.726375 63.95825) (end 175.726375 65.42075) (width 0.2) (layer "F.Cu") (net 4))
 (segment (start 73.28 66) (end 73.24 65.96) (width 0.4) (layer "F.Cu") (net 4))
 (segment (start 173.226375 65.42075) (end 175.726375 65.42075) (width 0.2) (layer "F.Cu") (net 4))
 (segment (start 165.194375 64.5) (end 164.925625 64.23125) (width 0.2) (layer "F.Cu") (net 4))
 (segment (start 175.726375 65.42075) (end 181.226375 65.42075) (width 0.2) (layer "F.Cu") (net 4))
 (segment (start 84.5775 59.04) (end 84.5375 59) (width 0.4) (layer "F.Cu") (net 4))
 (segment (start 78.5 66) (end 73.28 66) (width 0.4) (layer "F.Cu") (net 4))
 (segment (start 171.805625 64.5) (end 165.194375 64.5) (width 0.2) (layer "F.Cu") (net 4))
 (segment (start 175.184625 64.5) (end 175.726375 63.95825) (width 0.2) (layer "F.Cu") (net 4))
 (via (at 173.226375 52.8415) (size 0.6) (drill 0.3) (layers "F.Cu" "B.Cu") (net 4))
 (via (at 173.226375 63.42075) (size 0.6) (drill 0.3) (layers "F.Cu" "B.Cu") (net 4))
 (segment (start 173.226375 52.8415) (end 173.226375 63.42075) (width 0.2) (layer "B.Cu") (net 4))
 (segment (start 60 73) (end 59.42 73.58) (width 0.4) (layer "F.Cu") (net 5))
 (segment (start 60.5 56.5) (end 60 57) (width 0.4) (layer "F.Cu") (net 5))
 (segment (start 60 57) (end 60 73) (width 0.4) (layer "F.Cu") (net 5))
 (segment (start 59.42 73.58) (end 58 73.58) (width 0.4) (layer "F.Cu") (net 5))
 (segment (start 87.5 56.5) (end 60.5 56.5) (width 0.4) (layer "F.Cu") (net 5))
 (segment (start 57.92 73.5) (end 58 73.58) (width 0.2) (layer "F.Cu") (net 5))
 (segment (start 59.04 53.96) (end 54.5 58.5) (width 0.4) (layer "F.Cu") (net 6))
 (segment (start 87.5 53.96) (end 59.04 53.96) (width 0.4) (layer "F.Cu") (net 6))
 (segment (start 54.5 71) (end 57.96 71) (width 0.4) (layer "F.Cu") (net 6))
 (segment (start 57.96 71) (end 58 71.04) (width 0.4) (layer "F.Cu") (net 6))
 (segment (start 87.5 53.96) (end 87.54 54) (width 0.2) (layer "F.Cu") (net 6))
 (segment (start 54.5 58.5) (end 54.5 71) (width 0.4) (layer "F.Cu") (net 6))
 (segment (start 185 64) (end 181.03975 67.96025) (width 0.2) (layer "F.Cu") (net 8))
 (segment (start 185 63) (end 185 64) (width 0.2) (layer "F.Cu") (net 8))
 (segment (start 184.88075 62.88075) (end 185 63) (width 0.2) (layer "F.Cu") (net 8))
 (segment (start 181.03975 67.96025) (end 153.414625 67.96025) (width 0.2) (layer "F.Cu") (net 8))
 (segment (start 181.226375 62.88075) (end 184.88075 62.88075) (width 0.2) (layer "F.Cu") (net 8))
 (segment (start 153.414625 67.96025) (end 149.685625 64.23125) (width 0.2) (layer "F.Cu") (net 8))
 (segment (start 58 81) (end 59 81) (width 0.4) (layer "F.Cu") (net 23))
 (segment (start 58 76.12) (end 58 81) (width 0.4) (layer "F.Cu") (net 23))
 (segment (start 61.05 81) (end 66 81) (width 0.4) (layer "F.Cu") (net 18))
 (segment (start 73.36 76) (end 78.5 76) (width 0.4) (layer "F.Cu") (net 28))
 (segment (start 83.5 76) (end 84 75.5) (width 0.4) (layer "F.Cu") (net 28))
 (segment (start 78.5 76) (end 83.5 76) (width 0.4) (layer "F.Cu") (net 28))
 (segment (start 73.24 76.12) (end 73.36 76) (width 0.4) (layer "F.Cu") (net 28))
 (segment (start 153.726375 55.1105) (end 149.685625 59.15125) (width 0.2) (layer "F.Cu") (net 2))
 (segment (start 153.726375 48.3415) (end 153.726375 55.1105) (width 0.2) (layer "F.Cu") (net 2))
 (segment (start 153.726375 48.3415) (end 153.726375 45.8415) (width 0.2) (layer "F.Cu") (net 2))
 (segment (start 154.241375 45.3565) (end 172.726375 45.3565) (width 0.2) (layer "F.Cu") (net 2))
 (segment (start 153.643875 48.424) (end 153.726375 48.3415) (width 0.2) (layer "F.Cu") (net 2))
 (segment (start 153.726375 45.8415) (end 154.226375 45.3415) (width 0.2) (layer "F.Cu") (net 2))
 (segment (start 154.226375 45.3415) (end 154.241375 45.3565) (width 0.2) (layer "F.Cu") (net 2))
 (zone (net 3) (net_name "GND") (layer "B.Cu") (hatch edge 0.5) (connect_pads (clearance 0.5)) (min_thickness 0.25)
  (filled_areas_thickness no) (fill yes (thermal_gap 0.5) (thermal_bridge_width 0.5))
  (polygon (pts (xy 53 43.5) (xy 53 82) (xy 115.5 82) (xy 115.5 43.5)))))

